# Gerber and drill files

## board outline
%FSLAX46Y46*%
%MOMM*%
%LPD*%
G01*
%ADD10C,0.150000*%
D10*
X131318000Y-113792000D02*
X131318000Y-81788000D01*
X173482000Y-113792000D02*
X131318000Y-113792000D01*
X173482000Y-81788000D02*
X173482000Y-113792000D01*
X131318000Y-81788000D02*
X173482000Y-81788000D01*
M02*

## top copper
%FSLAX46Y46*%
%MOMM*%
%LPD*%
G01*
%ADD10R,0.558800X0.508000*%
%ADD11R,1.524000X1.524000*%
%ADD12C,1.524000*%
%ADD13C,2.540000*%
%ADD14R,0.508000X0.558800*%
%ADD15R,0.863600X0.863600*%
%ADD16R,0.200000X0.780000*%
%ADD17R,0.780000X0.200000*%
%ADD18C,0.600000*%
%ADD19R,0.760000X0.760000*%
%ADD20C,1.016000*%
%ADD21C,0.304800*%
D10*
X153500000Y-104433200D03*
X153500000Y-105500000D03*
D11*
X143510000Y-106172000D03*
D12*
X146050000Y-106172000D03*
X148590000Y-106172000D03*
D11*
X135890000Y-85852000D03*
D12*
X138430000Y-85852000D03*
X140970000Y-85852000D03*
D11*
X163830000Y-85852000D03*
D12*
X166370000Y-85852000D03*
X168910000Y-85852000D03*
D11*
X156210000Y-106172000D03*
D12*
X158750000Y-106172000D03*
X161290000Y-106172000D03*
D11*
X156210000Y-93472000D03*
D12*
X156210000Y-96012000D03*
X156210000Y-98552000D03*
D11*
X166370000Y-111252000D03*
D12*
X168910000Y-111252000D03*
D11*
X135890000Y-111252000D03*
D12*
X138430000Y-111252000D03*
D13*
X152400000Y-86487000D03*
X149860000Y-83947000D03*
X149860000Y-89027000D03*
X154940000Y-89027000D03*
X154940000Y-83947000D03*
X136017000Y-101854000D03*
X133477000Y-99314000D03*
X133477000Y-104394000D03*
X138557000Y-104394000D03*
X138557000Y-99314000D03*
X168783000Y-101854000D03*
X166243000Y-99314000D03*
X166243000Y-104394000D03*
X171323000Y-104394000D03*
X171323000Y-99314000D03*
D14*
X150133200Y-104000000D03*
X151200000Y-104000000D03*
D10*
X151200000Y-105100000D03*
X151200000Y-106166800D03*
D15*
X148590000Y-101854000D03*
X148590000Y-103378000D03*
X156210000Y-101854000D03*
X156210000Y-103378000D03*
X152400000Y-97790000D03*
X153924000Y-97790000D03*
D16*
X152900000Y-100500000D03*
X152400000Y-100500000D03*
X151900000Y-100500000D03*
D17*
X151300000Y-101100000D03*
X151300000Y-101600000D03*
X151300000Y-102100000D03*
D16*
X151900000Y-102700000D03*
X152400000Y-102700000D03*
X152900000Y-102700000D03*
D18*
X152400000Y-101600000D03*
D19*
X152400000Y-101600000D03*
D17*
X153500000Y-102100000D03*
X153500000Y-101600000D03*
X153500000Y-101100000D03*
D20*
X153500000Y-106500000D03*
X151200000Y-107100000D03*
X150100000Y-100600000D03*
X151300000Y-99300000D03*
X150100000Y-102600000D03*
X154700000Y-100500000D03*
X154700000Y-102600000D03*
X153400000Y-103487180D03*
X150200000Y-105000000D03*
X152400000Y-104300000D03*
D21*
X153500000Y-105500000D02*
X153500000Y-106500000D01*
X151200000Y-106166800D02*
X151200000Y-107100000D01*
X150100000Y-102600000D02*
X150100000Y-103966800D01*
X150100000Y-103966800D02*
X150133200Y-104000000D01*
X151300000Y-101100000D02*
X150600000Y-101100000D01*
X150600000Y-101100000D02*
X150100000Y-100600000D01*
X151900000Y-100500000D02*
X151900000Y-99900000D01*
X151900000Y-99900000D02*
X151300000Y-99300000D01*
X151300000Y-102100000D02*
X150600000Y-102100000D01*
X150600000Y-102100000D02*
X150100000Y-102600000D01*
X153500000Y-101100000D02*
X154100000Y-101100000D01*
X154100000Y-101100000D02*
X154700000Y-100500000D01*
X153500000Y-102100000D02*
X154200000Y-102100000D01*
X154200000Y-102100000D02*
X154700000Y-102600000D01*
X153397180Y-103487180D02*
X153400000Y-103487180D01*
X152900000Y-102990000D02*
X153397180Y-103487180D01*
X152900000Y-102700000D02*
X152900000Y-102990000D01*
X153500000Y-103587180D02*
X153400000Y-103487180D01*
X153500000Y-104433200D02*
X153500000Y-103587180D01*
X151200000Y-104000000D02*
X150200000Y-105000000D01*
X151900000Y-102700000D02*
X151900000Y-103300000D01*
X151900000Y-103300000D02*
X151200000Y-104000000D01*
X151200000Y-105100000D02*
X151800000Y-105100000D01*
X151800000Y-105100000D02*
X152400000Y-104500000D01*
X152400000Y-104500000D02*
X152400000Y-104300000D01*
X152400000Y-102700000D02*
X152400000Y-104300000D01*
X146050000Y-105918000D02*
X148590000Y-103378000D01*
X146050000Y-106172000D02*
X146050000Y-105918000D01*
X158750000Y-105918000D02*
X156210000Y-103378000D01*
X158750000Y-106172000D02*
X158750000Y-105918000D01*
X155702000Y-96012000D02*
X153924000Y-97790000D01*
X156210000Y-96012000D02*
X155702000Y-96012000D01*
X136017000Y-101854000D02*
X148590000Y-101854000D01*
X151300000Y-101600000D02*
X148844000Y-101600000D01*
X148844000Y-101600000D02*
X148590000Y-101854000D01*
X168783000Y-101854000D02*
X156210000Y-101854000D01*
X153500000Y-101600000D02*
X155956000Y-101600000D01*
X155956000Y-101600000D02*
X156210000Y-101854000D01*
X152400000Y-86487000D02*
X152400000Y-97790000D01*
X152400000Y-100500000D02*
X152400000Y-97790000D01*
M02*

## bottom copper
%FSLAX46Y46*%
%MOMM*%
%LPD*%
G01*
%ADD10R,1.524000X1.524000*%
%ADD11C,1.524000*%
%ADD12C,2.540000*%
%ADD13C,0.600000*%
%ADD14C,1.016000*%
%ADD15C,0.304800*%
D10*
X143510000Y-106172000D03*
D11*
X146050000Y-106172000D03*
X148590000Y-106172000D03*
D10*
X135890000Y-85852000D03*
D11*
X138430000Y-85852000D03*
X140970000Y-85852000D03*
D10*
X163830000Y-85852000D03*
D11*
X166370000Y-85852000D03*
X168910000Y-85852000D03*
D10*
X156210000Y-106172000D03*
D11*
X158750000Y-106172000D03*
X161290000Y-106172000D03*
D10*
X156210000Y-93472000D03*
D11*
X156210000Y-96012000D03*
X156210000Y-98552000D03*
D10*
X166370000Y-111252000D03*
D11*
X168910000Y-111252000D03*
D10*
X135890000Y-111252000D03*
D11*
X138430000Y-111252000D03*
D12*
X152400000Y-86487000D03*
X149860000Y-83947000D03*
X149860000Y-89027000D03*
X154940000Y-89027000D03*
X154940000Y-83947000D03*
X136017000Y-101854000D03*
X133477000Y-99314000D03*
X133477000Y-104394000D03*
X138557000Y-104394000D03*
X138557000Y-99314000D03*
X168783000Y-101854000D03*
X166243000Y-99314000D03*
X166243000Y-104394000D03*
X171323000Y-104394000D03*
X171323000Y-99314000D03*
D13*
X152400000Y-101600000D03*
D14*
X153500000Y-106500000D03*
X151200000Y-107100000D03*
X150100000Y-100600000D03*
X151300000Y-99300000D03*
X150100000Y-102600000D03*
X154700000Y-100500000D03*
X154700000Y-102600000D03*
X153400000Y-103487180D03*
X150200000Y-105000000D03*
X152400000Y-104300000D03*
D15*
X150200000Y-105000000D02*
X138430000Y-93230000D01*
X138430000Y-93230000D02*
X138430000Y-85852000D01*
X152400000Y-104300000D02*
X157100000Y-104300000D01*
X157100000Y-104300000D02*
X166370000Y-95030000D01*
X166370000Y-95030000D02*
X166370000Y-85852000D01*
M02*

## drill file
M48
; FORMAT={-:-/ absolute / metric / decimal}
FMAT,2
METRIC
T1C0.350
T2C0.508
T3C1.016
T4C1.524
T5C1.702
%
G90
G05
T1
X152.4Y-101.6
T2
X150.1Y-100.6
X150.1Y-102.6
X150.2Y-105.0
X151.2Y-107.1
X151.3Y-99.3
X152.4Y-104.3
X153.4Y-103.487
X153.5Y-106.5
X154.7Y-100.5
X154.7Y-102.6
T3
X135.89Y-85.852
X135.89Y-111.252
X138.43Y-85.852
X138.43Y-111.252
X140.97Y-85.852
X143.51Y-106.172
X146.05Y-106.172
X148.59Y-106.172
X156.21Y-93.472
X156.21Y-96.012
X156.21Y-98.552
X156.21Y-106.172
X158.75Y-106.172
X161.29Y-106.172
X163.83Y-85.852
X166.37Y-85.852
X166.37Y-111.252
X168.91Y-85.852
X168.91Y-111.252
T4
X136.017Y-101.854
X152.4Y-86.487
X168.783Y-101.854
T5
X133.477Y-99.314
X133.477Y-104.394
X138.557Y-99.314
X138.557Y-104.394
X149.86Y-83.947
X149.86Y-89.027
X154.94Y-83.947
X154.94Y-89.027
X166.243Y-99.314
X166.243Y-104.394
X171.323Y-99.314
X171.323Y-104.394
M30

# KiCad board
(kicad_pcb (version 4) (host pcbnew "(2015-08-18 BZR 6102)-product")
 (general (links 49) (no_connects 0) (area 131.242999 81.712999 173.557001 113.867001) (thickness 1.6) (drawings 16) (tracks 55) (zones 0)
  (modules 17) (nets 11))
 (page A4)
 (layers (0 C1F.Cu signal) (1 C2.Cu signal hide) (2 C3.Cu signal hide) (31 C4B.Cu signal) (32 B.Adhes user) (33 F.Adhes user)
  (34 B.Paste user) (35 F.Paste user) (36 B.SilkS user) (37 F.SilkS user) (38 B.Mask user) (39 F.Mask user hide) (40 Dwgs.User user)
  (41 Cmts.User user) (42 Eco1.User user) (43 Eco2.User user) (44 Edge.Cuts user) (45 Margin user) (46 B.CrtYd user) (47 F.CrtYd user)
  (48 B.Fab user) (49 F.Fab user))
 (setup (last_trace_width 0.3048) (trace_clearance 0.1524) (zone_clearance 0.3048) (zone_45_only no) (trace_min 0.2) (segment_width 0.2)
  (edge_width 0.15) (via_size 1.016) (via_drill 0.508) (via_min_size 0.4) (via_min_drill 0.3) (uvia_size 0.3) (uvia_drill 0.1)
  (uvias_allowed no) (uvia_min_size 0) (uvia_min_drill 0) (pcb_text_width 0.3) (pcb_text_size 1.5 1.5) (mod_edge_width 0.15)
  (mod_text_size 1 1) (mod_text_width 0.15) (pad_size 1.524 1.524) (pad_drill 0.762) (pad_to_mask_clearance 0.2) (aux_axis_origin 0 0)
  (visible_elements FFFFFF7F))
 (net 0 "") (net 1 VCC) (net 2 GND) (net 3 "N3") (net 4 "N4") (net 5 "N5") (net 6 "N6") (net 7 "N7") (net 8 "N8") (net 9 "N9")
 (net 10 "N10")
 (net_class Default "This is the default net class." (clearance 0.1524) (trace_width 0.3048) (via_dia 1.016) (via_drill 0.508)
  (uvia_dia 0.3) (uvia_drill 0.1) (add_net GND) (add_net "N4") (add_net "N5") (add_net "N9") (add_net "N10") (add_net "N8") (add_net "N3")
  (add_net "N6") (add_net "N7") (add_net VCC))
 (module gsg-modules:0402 (layer C1F.Cu) (at 153.5 104.9666 90) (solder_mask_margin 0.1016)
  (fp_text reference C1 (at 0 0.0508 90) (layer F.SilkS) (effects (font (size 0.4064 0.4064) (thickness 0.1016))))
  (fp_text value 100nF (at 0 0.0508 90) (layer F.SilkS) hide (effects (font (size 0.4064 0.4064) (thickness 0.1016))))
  (pad 2 smd rect (at 0.5334 0 90) (size 0.508 0.5588) (layers C1F.Cu F.Paste F.Mask) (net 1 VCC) (solder_mask_margin 0.1016))
  (pad 1 smd rect (at -0.5334 0 90) (size 0.508 0.5588) (layers C1F.Cu F.Paste F.Mask) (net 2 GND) (solder_mask_margin 0.1016)))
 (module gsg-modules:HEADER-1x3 (layer C1F.Cu) (at 146.05 106.172)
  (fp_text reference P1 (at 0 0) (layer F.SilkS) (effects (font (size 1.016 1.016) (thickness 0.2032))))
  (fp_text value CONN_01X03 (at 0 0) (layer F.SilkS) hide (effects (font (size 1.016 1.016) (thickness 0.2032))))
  (pad 1 thru_hole rect (at -2.54 0) (size 1.524 1.524) (drill 1.016) (layers *.Cu *.Mask F.SilkS) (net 2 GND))
  (pad 2 thru_hole circle (at 0 0) (size 1.524 1.524) (drill 1.016) (layers *.Cu *.Mask F.SilkS) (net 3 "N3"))
  (pad 3 thru_hole circle (at 2.54 0) (size 1.524 1.524) (drill 1.016) (layers *.Cu *.Mask F.SilkS) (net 1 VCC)))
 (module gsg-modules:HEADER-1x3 (layer C1F.Cu) (at 138.43 85.852)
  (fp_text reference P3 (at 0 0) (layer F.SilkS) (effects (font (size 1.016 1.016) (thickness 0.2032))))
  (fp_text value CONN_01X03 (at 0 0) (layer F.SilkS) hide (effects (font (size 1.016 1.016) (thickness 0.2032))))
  (pad 1 thru_hole rect (at -2.54 0) (size 1.524 1.524) (drill 1.016) (layers *.Cu *.Mask F.SilkS) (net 2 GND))
  (pad 2 thru_hole circle (at 0 0) (size 1.524 1.524) (drill 1.016) (layers *.Cu *.Mask F.SilkS) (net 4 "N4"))
  (pad 3 thru_hole circle (at 2.54 0) (size 1.524 1.524) (drill 1.016) (layers *.Cu *.Mask F.SilkS) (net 1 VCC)))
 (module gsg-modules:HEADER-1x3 (layer C1F.Cu) (at 166.37 85.852)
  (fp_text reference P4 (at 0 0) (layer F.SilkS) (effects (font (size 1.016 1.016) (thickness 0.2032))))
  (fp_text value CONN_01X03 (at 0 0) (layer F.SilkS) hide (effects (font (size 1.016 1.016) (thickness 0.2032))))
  (pad 1 thru_hole rect (at -2.54 0) (size 1.524 1.524) (drill 1.016) (layers *.Cu *.Mask F.SilkS) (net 2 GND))
  (pad 2 thru_hole circle (at 0 0) (size 1.524 1.524) (drill 1.016) (layers *.Cu *.Mask F.SilkS) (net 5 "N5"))
  (pad 3 thru_hole circle (at 2.54 0) (size 1.524 1.524) (drill 1.016) (layers *.Cu *.Mask F.SilkS) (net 1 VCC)))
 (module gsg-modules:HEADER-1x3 (layer C1F.Cu) (at 158.75 106.172)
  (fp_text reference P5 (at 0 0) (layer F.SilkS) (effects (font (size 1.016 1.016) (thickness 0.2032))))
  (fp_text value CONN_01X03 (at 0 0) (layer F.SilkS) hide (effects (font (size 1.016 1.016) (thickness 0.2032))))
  (pad 1 thru_hole rect (at -2.54 0) (size 1.524 1.524) (drill 1.016) (layers *.Cu *.Mask F.SilkS) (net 2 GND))
  (pad 2 thru_hole circle (at 0 0) (size 1.524 1.524) (drill 1.016) (layers *.Cu *.Mask F.SilkS) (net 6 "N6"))
  (pad 3 thru_hole circle (at 2.54 0) (size 1.524 1.524) (drill 1.016) (layers *.Cu *.Mask F.SilkS) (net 1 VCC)))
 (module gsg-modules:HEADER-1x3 (layer C1F.Cu) (at 156.21 96.012 270)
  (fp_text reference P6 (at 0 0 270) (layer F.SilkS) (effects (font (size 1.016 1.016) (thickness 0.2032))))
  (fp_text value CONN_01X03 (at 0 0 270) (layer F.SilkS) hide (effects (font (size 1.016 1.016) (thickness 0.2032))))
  (pad 1 thru_hole rect (at -2.54 0 270) (size 1.524 1.524) (drill 1.016) (layers *.Cu *.Mask F.SilkS) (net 2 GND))
  (pad 2 thru_hole circle (at 0 0 270) (size 1.524 1.524) (drill 1.016) (layers *.Cu *.Mask F.SilkS) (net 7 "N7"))
  (pad 3 thru_hole circle (at 2.54 0 270) (size 1.524 1.524) (drill 1.016) (layers *.Cu *.Mask F.SilkS) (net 1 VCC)))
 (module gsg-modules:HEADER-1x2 (layer C1F.Cu) (at 167.64 111.252)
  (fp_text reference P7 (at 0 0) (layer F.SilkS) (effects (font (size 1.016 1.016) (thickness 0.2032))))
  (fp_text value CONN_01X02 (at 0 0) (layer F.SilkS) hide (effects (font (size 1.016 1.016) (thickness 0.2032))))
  (pad 1 thru_hole rect (at -1.27 0) (size 1.524 1.524) (drill 1.016) (layers *.Cu *.Mask F.SilkS) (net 1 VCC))
  (pad 2 thru_hole circle (at 1.27 0) (size 1.524 1.524) (drill 1.016) (layers *.Cu *.Mask F.SilkS) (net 1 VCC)))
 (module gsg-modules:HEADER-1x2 (layer C1F.Cu) (at 137.16 111.252)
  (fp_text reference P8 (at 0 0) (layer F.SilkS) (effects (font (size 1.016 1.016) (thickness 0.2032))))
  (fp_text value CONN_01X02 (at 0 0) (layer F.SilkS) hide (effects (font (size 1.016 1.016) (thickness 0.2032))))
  (pad 1 thru_hole rect (at -1.27 0) (size 1.524 1.524) (drill 1.016) (layers *.Cu *.Mask F.SilkS) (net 2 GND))
  (pad 2 thru_hole circle (at 1.27 0) (size 1.524 1.524) (drill 1.016) (layers *.Cu *.Mask F.SilkS) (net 2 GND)))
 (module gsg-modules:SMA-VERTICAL (layer C1F.Cu) (at 152.4 86.487)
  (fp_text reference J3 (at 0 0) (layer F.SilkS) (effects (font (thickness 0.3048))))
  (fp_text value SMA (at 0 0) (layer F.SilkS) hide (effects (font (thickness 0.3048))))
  (pad 1 thru_hole circle (at 0 0) (size 2.54 2.54) (drill 1.524) (layers *.Cu *.Mask F.SilkS) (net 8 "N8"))
  (pad 2 thru_hole circle (at -2.54 -2.54) (size 2.54 2.54) (drill 1.7018) (layers *.Cu *.Mask F.SilkS) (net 2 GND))
  (pad 2 thru_hole circle (at -2.54 2.54) (size 2.54 2.54) (drill 1.7018) (layers *.Cu *.Mask F.SilkS) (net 2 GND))
  (pad 2 thru_hole circle (at 2.54 2.54) (size 2.54 2.54) (drill 1.7018) (layers *.Cu *.Mask F.SilkS) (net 2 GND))
  (pad 2 thru_hole circle (at 2.54 -2.54) (size 2.54 2.54) (drill 1.7018) (layers *.Cu *.Mask F.SilkS) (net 2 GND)))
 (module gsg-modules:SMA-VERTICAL (layer C1F.Cu) (at 136.017 101.854)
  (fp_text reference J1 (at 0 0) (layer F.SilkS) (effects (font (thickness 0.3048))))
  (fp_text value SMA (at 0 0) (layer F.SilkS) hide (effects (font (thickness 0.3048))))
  (pad 1 thru_hole circle (at 0 0) (size 2.54 2.54) (drill 1.524) (layers *.Cu *.Mask F.SilkS) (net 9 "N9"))
  (pad 2 thru_hole circle (at -2.54 -2.54) (size 2.54 2.54) (drill 1.7018) (layers *.Cu *.Mask F.SilkS) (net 2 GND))
  (pad 2 thru_hole circle (at -2.54 2.54) (size 2.54 2.54) (drill 1.7018) (layers *.Cu *.Mask F.SilkS) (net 2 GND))
  (pad 2 thru_hole circle (at 2.54 2.54) (size 2.54 2.54) (drill 1.7018) (layers *.Cu *.Mask F.SilkS) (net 2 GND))
  (pad 2 thru_hole circle (at 2.54 -2.54) (size 2.54 2.54) (drill 1.7018) (layers *.Cu *.Mask F.SilkS) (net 2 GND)))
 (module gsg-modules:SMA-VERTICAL (layer C1F.Cu) (at 168.783 101.854)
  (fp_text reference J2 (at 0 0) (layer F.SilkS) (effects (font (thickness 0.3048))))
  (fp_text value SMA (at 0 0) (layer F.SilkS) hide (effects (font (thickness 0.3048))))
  (pad 1 thru_hole circle (at 0 0) (size 2.54 2.54) (drill 1.524) (layers *.Cu *.Mask F.SilkS) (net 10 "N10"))
  (pad 2 thru_hole circle (at -2.54 -2.54) (size 2.54 2.54) (drill 1.7018) (layers *.Cu *.Mask F.SilkS) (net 2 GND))
  (pad 2 thru_hole circle (at -2.54 2.54) (size 2.54 2.54) (drill 1.7018) (layers *.Cu *.Mask F.SilkS) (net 2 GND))
  (pad 2 thru_hole circle (at 2.54 2.54) (size 2.54 2.54) (drill 1.7018) (layers *.Cu *.Mask F.SilkS) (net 2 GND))
  (pad 2 thru_hole circle (at 2.54 -2.54) (size 2.54 2.54) (drill 1.7018) (layers *.Cu *.Mask F.SilkS) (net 2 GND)))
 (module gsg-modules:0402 (layer C1F.Cu) (at 150.6666 104 180) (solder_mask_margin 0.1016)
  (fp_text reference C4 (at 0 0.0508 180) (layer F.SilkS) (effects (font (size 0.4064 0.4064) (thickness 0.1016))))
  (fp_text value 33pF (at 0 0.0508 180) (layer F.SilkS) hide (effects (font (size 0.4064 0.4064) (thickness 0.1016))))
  (pad 2 smd rect (at 0.5334 0 180) (size 0.508 0.5588) (layers C1F.Cu F.Paste F.Mask) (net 2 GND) (solder_mask_margin 0.1016))
  (pad 1 smd rect (at -0.5334 0 180) (size 0.508 0.5588) (layers C1F.Cu F.Paste F.Mask) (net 4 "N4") (solder_mask_margin 0.1016)))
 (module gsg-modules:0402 (layer C1F.Cu) (at 151.2 105.6334 90) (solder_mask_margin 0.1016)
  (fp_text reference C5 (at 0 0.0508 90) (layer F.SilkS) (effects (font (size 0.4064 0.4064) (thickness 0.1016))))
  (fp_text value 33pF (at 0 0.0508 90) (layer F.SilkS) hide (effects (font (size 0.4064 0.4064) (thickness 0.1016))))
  (pad 2 smd rect (at 0.5334 0 90) (size 0.508 0.5588) (layers C1F.Cu F.Paste F.Mask) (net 5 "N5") (solder_mask_margin 0.1016))
  (pad 1 smd rect (at -0.5334 0 90) (size 0.508 0.5588) (layers C1F.Cu F.Paste F.Mask) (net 2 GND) (solder_mask_margin 0.1016)))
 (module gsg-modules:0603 (layer C1F.Cu) (at 148.59 102.616 90) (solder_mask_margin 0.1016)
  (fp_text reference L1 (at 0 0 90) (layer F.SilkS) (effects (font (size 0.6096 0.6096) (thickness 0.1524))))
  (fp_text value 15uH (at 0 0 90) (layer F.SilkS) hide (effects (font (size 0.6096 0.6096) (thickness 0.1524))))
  (pad 2 smd rect (at 0.762 0 90) (size 0.8636 0.8636) (layers C1F.Cu F.Paste F.Mask) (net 9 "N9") (solder_mask_margin 0.1016)
   (clearance 0.1778))
  (pad 1 smd rect (at -0.762 0 90) (size 0.8636 0.8636) (layers C1F.Cu F.Paste F.Mask) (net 3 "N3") (solder_mask_margin 0.1016)
   (clearance 0.1778)))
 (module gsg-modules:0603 (layer C1F.Cu) (at 156.21 102.616 90) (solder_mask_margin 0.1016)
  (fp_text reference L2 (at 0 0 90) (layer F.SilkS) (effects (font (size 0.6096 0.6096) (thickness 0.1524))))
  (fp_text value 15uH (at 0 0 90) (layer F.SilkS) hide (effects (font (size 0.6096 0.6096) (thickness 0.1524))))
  (pad 2 smd rect (at 0.762 0 90) (size 0.8636 0.8636) (layers C1F.Cu F.Paste F.Mask) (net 10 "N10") (solder_mask_margin 0.1016)
   (clearance 0.1778))
  (pad 1 smd rect (at -0.762 0 90) (size 0.8636 0.8636) (layers C1F.Cu F.Paste F.Mask) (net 6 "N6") (solder_mask_margin 0.1016)
   (clearance 0.1778)))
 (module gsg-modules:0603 (layer C1F.Cu) (at 153.162 97.79 180) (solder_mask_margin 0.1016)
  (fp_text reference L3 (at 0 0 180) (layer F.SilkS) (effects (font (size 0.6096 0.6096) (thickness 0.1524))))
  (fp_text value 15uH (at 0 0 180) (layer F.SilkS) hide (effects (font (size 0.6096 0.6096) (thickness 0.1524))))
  (pad 2 smd rect (at 0.762 0 180) (size 0.8636 0.8636) (layers C1F.Cu F.Paste F.Mask) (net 8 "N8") (solder_mask_margin 0.1016)
   (clearance 0.1778))
  (pad 1 smd rect (at -0.762 0 180) (size 0.8636 0.8636) (layers C1F.Cu F.Paste F.Mask) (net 7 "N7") (solder_mask_margin 0.1016)
   (clearance 0.1778)))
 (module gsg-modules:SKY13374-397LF (layer C1F.Cu) (at 152.4 101.6 270) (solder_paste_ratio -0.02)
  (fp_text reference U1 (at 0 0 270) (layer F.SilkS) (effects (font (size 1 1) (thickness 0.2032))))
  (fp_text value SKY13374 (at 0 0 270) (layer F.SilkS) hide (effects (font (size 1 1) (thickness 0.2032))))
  (pad 1 smd rect (at -1.1 -0.5 270) (size 0.78 0.2) (layers C1F.Cu F.Paste F.Mask))
  (pad 2 smd rect (at -1.1 0 270) (size 0.78 0.2) (layers C1F.Cu F.Paste F.Mask) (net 8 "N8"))
  (pad 3 smd rect (at -1.1 0.5 270) (size 0.78 0.2) (layers C1F.Cu F.Paste F.Mask) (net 2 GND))
  (pad 4 smd rect (at -0.5 1.1 270) (size 0.2 0.78) (layers C1F.Cu F.Paste F.Mask) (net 2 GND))
  (pad 5 smd rect (at 0 1.1 270) (size 0.2 0.78) (layers C1F.Cu F.Paste F.Mask) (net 9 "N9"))
  (pad 6 smd rect (at 0.5 1.1 270) (size 0.2 0.78) (layers C1F.Cu F.Paste F.Mask) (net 2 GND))
  (pad 7 smd rect (at 1.1 0.5 270) (size 0.78 0.2) (layers C1F.Cu F.Paste F.Mask) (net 4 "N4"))
  (pad 8 smd rect (at 1.1 0 270) (size 0.78 0.2) (layers C1F.Cu F.Paste F.Mask) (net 5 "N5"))
  (pad 9 smd rect (at 1.1 -0.5 270) (size 0.78 0.2) (layers C1F.Cu F.Paste F.Mask) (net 1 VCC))
  (pad 0 thru_hole circle (at 0 0 270) (size 0.6 0.6) (drill 0.35) (layers *.Cu B.Mask) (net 2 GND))
  (pad 0 smd rect (at 0 0 270) (size 0.76 0.76) (layers C1F.Cu F.Paste F.Mask) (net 2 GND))
  (pad 10 smd rect (at 0.5 -1.1 270) (size 0.2 0.78) (layers C1F.Cu F.Paste F.Mask) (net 2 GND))
  (pad 11 smd rect (at 0 -1.1 270) (size 0.2 0.78) (layers C1F.Cu F.Paste F.Mask) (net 10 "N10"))
  (pad 12 smd rect (at -0.5 -1.1 270) (size 0.2 0.78) (layers C1F.Cu F.Paste F.Mask) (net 2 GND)))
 (gr_line (start 131.318 113.792) (end 131.318 81.788) (angle 90) (layer Edge.Cuts) (width 0.15))
 (gr_line (start 173.482 113.792) (end 131.318 113.792) (angle 90) (layer Edge.Cuts) (width 0.15))
 (gr_line (start 173.482 81.788) (end 173.482 113.792) (angle 90) (layer Edge.Cuts) (width 0.15))
 (gr_line (start 131.318 81.788) (end 173.482 81.788) (angle 90) (layer Edge.Cuts) (width 0.15))
 (segment (start 153.5 105.5) (end 153.5 106.5) (width 0.3048) (layer C1F.Cu) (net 2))
 (via (at 153.5 106.5) (size 1.016) (drill 0.508) (layers C1F.Cu C4B.Cu) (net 2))
 (segment (start 151.2 106.1668) (end 151.2 107.1) (width 0.3048) (layer C1F.Cu) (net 2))
 (via (at 151.2 107.1) (size 1.016) (drill 0.508) (layers C1F.Cu C4B.Cu) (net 2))
 (segment (start 150.1 102.6) (end 150.1 103.9668) (width 0.3048) (layer C1F.Cu) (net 2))
 (segment (start 150.1 103.9668) (end 150.1332 104) (width 0.3048) (layer C1F.Cu) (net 2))
 (segment (start 151.3 101.1) (end 150.6 101.1) (width 0.3048) (layer C1F.Cu) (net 2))
 (segment (start 150.6 101.1) (end 150.1 100.6) (width 0.3048) (layer C1F.Cu) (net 2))
 (via (at 150.1 100.6) (size 1.016) (drill 0.508) (layers C1F.Cu C4B.Cu) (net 2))
 (segment (start 151.9 100.5) (end 151.9 99.9) (width 0.3048) (layer C1F.Cu) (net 2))
 (segment (start 151.9 99.9) (end 151.3 99.3) (width 0.3048) (layer C1F.Cu) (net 2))
 (via (at 151.3 99.3) (size 1.016) (drill 0.508) (layers C1F.Cu C4B.Cu) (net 2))
 (segment (start 151.3 102.1) (end 150.6 102.1) (width 0.3048) (layer C1F.Cu) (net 2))
 (segment (start 150.6 102.1) (end 150.1 102.6) (width 0.3048) (layer C1F.Cu) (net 2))
 (via (at 150.1 102.6) (size 1.016) (drill 0.508) (layers C1F.Cu C4B.Cu) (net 2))
 (segment (start 153.5 101.1) (end 154.1 101.1) (width 0.3048) (layer C1F.Cu) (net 2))
 (segment (start 154.1 101.1) (end 154.7 100.5) (width 0.3048) (layer C1F.Cu) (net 2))
 (via (at 154.7 100.5) (size 1.016) (drill 0.508) (layers C1F.Cu C4B.Cu) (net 2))
 (segment (start 153.5 102.1) (end 154.2 102.1) (width 0.3048) (layer C1F.Cu) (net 2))
 (segment (start 154.2 102.1) (end 154.7 102.6) (width 0.3048) (layer C1F.Cu) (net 2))
 (via (at 154.7 102.6) (size 1.016) (drill 0.508) (layers C1F.Cu C4B.Cu) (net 2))
 (segment (start 153.39718 103.48718) (end 153.4 103.48718) (width 0.3048) (layer C1F.Cu) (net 1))
 (segment (start 152.9 102.99) (end 153.39718 103.48718) (width 0.3048) (layer C1F.Cu) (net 1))
 (segment (start 152.9 102.7) (end 152.9 102.99) (width 0.3048) (layer C1F.Cu) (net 1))
 (segment (start 153.5 103.58718) (end 153.4 103.48718) (width 0.3048) (layer C1F.Cu) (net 1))
 (segment (start 153.5 104.4332) (end 153.5 103.58718) (width 0.3048) (layer C1F.Cu) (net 1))
 (via (at 153.4 103.48718) (size 1.016) (drill 0.508) (layers C1F.Cu C4B.Cu) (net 1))
 (segment (start 150.2 105) (end 138.43 93.23) (width 0.3048) (layer C4B.Cu) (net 4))
 (segment (start 138.43 93.23) (end 138.43 85.852) (width 0.3048) (layer C4B.Cu) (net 4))
 (segment (start 151.2 104) (end 150.2 105) (width 0.3048) (layer C1F.Cu) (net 4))
 (via (at 150.2 105) (size 1.016) (drill 0.508) (layers C1F.Cu C4B.Cu) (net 4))
 (segment (start 151.9 102.7) (end 151.9 103.3) (width 0.3048) (layer C1F.Cu) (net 4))
 (segment (start 151.9 103.3) (end 151.2 104) (width 0.3048) (layer C1F.Cu) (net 4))
 (segment (start 151.2 105.1) (end 151.8 105.1) (width 0.3048) (layer C1F.Cu) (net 5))
 (segment (start 151.8 105.1) (end 152.4 104.5) (width 0.3048) (layer C1F.Cu) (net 5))
 (segment (start 152.4 104.5) (end 152.4 104.3) (width 0.3048) (layer C1F.Cu) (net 5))
 (segment (start 152.4 104.3) (end 157.1 104.3) (width 0.3048) (layer C4B.Cu) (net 5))
 (segment (start 157.1 104.3) (end 166.37 95.03) (width 0.3048) (layer C4B.Cu) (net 5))
 (segment (start 166.37 95.03) (end 166.37 85.852) (width 0.3048) (layer C4B.Cu) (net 5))
 (segment (start 152.4 102.7) (end 152.4 104.3) (width 0.3048) (layer C1F.Cu) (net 5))
 (via (at 152.4 104.3) (size 1.016) (drill 0.508) (layers C1F.Cu C4B.Cu) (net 5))
 (segment (start 146.05 105.918) (end 148.59 103.378) (width 0.3048) (layer C1F.Cu) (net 3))
 (segment (start 146.05 106.172) (end 146.05 105.918) (width 0.3048) (layer C1F.Cu) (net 3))
 (segment (start 158.75 105.918) (end 156.21 103.378) (width 0.3048) (layer C1F.Cu) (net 6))
 (segment (start 158.75 106.172) (end 158.75 105.918) (width 0.3048) (layer C1F.Cu) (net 6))
 (segment (start 155.702 96.012) (end 153.924 97.79) (width 0.3048) (layer C1F.Cu) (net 7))
 (segment (start 156.21 96.012) (end 155.702 96.012) (width 0.3048) (layer C1F.Cu) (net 7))
 (segment (start 136.017 101.854) (end 148.59 101.854) (width 0.3048) (layer C1F.Cu) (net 9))
 (segment (start 151.3 101.6) (end 148.844 101.6) (width 0.3048) (layer C1F.Cu) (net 9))
 (segment (start 148.844 101.6) (end 148.59 101.854) (width 0.3048) (layer C1F.Cu) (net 9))
 (segment (start 168.783 101.854) (end 156.21 101.854) (width 0.3048) (layer C1F.Cu) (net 10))
 (segment (start 153.5 101.6) (end 155.956 101.6) (width 0.3048) (layer C1F.Cu) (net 10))
 (segment (start 155.956 101.6) (end 156.21 101.854) (width 0.3048) (layer C1F.Cu) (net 10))
 (segment (start 152.4 86.487) (end 152.4 97.79) (width 0.3048) (layer C1F.Cu) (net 8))
 (segment (start 152.4 100.5) (end 152.4 97.79) (width 0.3048) (layer C1F.Cu) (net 8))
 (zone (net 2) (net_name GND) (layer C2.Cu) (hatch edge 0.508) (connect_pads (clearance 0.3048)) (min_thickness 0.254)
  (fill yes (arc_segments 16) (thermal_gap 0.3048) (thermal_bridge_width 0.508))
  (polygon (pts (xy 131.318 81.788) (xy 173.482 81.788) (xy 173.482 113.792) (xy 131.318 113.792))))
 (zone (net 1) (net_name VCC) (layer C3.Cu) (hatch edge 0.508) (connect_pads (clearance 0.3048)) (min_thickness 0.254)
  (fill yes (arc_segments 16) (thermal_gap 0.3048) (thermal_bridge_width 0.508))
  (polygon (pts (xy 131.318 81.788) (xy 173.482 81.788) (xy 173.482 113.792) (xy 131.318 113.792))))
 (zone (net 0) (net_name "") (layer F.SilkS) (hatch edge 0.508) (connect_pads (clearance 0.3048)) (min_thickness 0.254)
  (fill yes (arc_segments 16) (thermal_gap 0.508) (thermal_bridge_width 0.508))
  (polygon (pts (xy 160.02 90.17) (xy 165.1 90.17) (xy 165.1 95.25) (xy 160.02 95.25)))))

